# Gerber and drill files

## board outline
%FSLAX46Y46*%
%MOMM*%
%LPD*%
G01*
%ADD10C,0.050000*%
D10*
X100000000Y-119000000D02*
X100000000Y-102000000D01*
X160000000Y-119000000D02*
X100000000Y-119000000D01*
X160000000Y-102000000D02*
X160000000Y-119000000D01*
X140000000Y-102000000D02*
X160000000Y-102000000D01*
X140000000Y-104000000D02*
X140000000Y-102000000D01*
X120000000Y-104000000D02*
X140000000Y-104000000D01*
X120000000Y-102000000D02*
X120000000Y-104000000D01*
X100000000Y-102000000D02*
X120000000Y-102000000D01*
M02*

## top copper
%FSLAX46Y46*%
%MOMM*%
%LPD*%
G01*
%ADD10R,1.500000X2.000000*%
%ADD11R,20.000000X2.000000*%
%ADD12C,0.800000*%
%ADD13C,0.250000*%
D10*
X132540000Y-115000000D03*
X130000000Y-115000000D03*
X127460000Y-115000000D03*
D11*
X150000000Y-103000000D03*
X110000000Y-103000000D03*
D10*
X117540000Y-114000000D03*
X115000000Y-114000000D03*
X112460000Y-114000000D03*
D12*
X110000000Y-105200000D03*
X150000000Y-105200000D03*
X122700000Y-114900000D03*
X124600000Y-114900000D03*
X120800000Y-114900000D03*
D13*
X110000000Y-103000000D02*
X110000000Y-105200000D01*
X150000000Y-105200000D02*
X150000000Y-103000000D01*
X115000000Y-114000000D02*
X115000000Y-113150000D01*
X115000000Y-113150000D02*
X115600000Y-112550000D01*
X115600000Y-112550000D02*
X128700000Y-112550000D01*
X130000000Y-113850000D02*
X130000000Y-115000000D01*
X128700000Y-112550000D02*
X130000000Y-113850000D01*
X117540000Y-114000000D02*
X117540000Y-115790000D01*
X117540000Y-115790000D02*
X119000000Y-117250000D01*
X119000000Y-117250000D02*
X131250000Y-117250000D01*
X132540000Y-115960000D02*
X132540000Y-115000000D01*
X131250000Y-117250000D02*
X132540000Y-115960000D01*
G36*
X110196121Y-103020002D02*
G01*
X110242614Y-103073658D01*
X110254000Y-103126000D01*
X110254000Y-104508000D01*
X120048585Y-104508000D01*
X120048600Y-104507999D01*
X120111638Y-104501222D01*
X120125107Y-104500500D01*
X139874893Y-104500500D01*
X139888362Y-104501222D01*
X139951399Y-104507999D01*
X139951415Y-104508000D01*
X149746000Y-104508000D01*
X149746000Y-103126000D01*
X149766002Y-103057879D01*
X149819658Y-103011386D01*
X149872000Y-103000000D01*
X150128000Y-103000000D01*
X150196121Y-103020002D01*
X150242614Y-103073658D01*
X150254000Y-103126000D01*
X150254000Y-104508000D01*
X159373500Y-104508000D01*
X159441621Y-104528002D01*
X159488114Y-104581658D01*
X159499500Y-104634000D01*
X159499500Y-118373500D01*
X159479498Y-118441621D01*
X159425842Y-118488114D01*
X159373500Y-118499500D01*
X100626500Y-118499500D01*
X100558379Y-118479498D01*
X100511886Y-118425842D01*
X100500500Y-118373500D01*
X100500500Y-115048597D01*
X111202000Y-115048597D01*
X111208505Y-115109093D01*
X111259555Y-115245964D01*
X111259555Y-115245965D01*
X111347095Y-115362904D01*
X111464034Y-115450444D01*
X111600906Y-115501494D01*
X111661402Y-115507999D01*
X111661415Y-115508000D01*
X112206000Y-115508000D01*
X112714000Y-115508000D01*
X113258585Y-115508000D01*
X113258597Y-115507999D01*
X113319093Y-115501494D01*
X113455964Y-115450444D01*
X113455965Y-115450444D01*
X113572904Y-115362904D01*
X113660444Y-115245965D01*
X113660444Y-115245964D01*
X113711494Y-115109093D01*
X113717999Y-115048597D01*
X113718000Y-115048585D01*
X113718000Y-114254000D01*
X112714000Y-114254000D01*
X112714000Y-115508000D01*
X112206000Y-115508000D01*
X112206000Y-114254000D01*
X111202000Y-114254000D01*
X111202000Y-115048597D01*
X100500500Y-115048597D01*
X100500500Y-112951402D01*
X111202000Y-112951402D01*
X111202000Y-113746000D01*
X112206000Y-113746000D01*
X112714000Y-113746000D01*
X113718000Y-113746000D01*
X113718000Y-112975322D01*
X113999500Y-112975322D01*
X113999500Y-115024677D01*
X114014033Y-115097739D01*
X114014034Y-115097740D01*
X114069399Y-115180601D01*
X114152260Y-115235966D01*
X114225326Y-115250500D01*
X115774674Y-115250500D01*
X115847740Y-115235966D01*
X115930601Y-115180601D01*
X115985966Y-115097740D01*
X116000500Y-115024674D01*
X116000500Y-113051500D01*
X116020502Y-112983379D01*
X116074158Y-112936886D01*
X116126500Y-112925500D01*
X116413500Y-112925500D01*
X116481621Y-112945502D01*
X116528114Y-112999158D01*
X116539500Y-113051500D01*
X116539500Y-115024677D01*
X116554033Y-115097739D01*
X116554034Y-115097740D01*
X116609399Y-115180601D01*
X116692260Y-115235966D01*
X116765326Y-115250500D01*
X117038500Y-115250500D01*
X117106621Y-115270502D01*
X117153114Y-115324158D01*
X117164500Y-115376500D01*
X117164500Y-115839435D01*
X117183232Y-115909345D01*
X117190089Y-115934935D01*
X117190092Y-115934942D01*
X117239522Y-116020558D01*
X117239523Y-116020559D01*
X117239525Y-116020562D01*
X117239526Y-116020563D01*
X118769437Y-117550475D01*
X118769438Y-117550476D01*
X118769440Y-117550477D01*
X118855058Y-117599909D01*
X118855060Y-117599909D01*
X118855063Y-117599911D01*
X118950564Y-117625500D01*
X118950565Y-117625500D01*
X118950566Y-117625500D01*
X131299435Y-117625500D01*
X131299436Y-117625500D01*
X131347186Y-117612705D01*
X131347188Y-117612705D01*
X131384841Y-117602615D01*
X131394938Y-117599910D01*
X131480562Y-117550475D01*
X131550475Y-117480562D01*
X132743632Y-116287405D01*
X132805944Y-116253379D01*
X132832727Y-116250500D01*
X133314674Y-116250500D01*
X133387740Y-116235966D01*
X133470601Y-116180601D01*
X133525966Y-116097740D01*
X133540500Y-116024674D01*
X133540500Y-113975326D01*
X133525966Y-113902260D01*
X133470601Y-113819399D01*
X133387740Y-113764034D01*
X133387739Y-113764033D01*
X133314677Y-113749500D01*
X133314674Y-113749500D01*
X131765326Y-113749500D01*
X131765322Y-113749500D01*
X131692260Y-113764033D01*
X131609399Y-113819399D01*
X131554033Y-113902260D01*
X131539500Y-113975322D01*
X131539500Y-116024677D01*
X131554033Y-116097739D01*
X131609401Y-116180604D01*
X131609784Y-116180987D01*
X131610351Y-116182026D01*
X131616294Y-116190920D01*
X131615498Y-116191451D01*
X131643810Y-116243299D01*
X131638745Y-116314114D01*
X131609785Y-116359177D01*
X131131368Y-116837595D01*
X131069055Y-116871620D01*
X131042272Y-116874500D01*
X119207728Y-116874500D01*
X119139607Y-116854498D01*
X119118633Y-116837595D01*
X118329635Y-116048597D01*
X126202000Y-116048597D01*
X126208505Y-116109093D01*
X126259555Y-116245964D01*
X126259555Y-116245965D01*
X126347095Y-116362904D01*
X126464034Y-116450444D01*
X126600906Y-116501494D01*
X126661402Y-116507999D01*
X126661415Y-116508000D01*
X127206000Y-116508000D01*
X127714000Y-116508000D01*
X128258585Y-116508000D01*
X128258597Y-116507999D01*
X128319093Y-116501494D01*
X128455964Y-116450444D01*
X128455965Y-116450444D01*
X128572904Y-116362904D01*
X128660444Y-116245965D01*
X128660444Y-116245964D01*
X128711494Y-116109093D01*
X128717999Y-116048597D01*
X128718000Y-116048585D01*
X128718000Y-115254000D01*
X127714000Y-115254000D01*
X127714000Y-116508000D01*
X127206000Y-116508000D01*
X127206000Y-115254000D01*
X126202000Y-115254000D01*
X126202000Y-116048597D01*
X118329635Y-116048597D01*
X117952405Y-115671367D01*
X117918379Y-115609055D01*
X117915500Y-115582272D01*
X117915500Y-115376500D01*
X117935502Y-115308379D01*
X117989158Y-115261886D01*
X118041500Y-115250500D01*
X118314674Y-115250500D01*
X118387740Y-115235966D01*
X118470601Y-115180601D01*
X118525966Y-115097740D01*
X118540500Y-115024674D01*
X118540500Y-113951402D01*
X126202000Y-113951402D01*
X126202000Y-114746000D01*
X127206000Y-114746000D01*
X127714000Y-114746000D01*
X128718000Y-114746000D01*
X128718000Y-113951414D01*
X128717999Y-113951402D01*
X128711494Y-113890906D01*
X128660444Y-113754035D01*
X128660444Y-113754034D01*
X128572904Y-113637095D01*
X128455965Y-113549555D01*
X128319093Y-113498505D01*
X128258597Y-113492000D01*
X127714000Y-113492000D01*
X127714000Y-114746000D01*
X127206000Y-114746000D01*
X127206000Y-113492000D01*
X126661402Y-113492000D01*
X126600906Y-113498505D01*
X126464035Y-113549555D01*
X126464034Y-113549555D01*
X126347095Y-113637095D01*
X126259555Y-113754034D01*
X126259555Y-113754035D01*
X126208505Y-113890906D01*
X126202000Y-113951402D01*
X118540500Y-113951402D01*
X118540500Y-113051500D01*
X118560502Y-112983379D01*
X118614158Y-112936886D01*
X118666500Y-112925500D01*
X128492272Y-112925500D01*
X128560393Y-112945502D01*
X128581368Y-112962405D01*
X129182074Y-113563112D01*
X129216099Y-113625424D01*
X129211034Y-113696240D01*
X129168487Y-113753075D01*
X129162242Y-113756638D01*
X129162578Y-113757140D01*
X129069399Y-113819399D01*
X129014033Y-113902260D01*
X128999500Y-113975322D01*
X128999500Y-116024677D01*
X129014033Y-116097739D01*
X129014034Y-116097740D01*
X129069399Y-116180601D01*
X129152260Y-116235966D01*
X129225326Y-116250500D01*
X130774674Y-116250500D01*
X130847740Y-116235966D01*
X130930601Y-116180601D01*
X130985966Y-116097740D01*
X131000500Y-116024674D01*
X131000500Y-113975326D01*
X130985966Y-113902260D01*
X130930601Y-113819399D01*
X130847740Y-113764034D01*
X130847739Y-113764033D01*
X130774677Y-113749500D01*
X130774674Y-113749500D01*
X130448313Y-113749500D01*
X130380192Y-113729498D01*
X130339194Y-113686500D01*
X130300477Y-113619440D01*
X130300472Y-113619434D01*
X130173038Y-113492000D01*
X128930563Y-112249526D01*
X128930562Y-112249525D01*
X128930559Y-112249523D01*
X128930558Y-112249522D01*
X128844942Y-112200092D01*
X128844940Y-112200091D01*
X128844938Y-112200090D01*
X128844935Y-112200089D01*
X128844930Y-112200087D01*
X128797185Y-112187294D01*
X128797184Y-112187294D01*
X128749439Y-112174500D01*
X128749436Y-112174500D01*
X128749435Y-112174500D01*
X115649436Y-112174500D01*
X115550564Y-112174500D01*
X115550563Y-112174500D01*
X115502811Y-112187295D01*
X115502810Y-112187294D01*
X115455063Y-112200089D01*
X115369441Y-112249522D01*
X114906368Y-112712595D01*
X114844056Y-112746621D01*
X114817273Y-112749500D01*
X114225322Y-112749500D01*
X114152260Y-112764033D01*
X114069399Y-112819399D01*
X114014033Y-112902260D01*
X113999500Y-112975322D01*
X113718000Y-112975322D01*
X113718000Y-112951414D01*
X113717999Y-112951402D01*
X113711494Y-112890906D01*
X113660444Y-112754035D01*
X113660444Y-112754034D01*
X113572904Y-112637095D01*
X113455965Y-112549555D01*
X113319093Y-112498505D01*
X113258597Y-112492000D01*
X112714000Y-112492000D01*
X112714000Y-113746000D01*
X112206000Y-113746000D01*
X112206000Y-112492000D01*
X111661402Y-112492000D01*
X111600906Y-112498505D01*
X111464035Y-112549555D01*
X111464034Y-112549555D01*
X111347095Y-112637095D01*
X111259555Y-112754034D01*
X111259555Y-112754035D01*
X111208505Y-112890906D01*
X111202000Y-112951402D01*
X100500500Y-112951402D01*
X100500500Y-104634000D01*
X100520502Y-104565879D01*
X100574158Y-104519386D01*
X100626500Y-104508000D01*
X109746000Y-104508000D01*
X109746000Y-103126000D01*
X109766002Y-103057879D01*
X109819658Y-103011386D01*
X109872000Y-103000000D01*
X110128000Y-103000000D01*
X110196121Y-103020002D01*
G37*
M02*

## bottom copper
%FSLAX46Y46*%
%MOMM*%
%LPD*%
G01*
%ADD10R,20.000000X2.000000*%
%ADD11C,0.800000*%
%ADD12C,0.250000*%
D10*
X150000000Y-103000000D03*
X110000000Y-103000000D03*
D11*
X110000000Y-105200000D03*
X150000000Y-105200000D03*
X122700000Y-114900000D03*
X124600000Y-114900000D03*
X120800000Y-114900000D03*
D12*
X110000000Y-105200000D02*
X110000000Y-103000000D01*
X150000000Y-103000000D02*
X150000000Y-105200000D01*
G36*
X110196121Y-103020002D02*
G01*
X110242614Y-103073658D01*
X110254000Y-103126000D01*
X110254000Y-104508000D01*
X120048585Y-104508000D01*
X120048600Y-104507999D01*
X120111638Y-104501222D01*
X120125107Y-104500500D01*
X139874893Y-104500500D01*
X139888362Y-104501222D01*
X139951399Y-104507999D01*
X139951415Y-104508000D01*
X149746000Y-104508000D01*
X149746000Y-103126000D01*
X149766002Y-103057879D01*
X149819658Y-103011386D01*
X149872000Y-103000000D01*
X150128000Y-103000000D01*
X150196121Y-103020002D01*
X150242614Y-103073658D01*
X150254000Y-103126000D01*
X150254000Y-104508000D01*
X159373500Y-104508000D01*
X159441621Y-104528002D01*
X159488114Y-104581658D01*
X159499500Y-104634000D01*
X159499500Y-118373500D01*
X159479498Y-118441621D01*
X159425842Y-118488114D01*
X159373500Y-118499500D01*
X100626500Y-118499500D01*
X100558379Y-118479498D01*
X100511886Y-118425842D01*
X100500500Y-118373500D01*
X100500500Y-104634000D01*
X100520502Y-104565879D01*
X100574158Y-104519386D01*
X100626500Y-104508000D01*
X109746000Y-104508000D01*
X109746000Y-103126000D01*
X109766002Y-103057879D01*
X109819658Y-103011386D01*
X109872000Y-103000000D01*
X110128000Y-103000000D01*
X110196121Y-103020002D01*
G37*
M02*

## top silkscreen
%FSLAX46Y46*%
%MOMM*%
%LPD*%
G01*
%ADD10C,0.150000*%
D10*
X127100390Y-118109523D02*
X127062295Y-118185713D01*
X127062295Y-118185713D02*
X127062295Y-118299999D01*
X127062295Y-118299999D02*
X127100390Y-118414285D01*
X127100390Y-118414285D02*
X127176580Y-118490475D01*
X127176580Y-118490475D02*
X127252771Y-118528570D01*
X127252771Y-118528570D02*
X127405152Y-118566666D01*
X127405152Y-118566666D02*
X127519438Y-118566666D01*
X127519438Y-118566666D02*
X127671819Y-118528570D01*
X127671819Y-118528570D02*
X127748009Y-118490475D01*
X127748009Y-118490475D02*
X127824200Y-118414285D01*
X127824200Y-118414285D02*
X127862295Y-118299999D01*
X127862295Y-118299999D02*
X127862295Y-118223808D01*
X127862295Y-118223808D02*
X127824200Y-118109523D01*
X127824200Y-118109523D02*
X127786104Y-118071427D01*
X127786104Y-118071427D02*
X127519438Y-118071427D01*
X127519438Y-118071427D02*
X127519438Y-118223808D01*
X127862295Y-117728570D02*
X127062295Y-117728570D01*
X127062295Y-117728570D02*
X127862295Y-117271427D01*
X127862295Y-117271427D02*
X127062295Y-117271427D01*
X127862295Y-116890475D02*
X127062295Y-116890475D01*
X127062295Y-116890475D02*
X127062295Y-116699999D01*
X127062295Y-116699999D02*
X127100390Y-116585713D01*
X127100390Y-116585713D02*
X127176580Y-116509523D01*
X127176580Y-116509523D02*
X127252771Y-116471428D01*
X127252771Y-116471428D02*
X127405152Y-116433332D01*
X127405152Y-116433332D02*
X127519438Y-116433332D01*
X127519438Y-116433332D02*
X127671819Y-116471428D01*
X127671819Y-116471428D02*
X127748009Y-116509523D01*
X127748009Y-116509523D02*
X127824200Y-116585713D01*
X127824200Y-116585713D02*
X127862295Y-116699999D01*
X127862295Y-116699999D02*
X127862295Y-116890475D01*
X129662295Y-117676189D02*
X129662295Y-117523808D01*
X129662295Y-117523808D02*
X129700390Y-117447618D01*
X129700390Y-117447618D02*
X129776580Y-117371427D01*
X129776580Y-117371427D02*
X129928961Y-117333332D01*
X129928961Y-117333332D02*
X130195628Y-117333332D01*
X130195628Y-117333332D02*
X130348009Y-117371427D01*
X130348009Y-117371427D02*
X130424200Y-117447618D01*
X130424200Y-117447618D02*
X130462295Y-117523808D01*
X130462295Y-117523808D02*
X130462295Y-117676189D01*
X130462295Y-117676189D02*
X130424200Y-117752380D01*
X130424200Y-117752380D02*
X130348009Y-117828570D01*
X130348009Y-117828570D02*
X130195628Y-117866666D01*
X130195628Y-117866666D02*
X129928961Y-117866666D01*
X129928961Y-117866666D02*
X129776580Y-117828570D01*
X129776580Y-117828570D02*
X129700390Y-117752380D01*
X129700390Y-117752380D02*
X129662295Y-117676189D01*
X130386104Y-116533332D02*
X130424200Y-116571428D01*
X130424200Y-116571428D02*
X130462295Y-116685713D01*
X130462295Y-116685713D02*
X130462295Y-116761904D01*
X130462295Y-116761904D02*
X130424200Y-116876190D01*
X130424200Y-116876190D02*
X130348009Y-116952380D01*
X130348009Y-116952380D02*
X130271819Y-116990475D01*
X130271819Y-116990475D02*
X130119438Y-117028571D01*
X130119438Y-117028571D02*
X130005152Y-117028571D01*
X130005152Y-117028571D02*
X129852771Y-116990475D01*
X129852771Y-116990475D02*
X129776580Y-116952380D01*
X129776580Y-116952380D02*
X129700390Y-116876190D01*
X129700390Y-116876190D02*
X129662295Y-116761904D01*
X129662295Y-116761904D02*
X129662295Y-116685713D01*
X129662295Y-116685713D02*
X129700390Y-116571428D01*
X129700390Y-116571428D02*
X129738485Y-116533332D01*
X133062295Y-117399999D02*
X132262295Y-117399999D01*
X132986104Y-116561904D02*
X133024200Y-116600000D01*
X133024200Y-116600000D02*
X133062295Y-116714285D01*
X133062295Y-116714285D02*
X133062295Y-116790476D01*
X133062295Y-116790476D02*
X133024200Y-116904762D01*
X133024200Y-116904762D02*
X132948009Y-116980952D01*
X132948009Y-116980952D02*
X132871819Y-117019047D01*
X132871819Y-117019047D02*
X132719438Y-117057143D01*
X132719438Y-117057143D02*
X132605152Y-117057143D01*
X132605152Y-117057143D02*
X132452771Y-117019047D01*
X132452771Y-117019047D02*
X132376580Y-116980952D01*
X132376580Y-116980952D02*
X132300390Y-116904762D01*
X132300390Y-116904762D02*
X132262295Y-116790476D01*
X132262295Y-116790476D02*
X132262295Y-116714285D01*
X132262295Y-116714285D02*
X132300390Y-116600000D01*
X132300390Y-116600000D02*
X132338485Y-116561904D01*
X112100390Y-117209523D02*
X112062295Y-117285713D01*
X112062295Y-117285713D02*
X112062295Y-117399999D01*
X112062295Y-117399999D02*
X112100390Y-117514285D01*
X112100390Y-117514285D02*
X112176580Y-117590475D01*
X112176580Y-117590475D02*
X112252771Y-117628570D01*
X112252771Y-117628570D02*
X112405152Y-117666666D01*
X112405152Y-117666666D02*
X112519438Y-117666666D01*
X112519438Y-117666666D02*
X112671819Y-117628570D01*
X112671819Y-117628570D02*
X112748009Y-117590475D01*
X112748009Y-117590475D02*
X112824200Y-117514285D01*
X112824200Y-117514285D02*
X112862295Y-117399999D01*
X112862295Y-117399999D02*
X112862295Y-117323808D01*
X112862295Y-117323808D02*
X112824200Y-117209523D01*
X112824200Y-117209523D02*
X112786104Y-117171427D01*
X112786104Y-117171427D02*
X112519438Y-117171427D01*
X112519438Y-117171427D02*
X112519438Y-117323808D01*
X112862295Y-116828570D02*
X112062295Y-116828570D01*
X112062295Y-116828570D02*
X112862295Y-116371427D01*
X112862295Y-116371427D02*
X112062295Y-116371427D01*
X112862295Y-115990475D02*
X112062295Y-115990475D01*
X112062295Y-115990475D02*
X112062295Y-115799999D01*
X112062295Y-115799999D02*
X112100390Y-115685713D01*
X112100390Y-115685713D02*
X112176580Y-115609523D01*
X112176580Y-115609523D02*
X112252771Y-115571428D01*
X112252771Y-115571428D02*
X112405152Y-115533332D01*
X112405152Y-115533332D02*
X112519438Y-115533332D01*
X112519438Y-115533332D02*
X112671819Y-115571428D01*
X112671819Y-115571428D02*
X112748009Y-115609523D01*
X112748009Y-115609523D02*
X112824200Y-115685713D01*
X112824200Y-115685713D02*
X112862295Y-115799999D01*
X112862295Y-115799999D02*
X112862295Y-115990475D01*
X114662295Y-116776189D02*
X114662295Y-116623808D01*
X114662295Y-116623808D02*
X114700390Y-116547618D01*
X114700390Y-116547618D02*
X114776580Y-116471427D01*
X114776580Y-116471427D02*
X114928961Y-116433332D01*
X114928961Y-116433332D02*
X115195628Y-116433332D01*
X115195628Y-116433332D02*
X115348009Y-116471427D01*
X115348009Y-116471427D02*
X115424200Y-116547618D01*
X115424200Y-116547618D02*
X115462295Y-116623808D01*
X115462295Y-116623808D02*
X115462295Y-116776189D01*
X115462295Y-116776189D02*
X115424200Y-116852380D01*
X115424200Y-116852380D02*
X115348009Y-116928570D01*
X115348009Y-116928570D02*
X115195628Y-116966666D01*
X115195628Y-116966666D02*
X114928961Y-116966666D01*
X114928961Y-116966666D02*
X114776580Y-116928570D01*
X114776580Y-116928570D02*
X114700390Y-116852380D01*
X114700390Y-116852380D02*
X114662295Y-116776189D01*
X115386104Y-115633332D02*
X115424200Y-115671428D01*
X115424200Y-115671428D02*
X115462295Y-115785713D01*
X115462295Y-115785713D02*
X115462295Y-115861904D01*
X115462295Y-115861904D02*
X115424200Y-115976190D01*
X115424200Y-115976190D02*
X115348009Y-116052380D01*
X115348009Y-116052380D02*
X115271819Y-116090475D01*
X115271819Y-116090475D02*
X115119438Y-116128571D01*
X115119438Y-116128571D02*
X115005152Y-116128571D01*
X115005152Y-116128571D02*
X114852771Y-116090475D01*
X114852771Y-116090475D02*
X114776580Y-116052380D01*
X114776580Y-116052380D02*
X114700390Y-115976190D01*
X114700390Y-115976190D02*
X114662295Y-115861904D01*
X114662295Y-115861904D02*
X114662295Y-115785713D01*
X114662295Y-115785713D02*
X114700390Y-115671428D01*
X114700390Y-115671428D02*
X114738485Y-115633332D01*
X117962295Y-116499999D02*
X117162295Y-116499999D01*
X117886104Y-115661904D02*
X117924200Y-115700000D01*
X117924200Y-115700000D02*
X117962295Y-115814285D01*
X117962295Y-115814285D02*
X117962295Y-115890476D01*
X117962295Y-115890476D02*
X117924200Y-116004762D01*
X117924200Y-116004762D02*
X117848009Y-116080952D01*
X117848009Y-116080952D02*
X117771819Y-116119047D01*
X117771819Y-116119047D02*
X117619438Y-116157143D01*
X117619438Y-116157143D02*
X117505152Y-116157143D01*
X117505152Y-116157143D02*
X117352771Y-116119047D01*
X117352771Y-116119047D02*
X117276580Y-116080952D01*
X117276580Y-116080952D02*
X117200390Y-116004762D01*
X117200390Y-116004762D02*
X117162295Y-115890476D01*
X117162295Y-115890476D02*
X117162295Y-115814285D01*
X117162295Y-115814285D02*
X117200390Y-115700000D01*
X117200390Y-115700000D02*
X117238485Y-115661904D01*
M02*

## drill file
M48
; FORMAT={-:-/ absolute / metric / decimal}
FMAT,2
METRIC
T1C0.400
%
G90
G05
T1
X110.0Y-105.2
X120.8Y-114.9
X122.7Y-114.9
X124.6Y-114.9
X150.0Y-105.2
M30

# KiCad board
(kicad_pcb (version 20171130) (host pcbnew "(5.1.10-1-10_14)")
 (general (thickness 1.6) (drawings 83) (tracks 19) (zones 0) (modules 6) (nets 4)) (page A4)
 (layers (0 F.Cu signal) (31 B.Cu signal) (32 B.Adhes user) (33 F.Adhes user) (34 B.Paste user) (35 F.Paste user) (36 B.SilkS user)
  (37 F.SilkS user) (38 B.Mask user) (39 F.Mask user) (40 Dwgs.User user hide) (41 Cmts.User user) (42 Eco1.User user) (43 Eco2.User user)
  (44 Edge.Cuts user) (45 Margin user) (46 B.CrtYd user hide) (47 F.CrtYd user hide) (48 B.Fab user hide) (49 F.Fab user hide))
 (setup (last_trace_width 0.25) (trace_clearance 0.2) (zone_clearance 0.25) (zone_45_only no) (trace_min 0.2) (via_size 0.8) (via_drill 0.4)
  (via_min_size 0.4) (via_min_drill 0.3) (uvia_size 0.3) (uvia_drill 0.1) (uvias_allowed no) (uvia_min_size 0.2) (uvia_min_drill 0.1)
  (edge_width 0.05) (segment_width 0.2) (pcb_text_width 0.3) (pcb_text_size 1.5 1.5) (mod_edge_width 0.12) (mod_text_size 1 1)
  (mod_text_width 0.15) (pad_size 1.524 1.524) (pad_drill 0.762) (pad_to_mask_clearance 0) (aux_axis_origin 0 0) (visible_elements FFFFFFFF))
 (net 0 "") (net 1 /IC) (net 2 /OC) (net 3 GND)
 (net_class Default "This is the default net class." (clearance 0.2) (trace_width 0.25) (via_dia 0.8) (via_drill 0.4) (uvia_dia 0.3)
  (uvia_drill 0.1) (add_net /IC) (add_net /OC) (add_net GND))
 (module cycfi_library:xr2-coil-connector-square (layer F.Cu) (at 130 115)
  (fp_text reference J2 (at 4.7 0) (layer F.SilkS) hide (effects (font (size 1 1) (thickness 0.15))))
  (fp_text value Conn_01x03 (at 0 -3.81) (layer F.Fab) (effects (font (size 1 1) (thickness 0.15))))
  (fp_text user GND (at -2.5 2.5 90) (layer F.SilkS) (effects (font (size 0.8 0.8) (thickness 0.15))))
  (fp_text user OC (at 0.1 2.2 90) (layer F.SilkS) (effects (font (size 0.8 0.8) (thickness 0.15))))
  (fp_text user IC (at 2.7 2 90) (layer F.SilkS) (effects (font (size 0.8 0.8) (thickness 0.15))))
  (pad 3 smd rect (at 2.54 0) (size 1.5 2) (layers F.Cu F.Paste F.Mask) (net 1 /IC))
  (pad 2 smd rect (at 0 0) (size 1.5 2) (layers F.Cu F.Paste F.Mask) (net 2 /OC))
  (pad 1 smd rect (at -2.54 0) (size 1.5 2) (layers F.Cu F.Paste F.Mask) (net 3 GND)))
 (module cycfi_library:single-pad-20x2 (layer B.Cu) (at 150 103)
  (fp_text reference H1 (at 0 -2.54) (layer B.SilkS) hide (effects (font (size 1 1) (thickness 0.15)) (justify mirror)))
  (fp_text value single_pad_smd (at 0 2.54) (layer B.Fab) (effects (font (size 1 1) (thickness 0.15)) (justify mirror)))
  (pad 1 smd rect (at 0 0) (size 20 2) (layers B.Cu B.Paste B.Mask) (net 3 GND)))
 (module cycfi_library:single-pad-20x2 (layer F.Cu) (at 150 103)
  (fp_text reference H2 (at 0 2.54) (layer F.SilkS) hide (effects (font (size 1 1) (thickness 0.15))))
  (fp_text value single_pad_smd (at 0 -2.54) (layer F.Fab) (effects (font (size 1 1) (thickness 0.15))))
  (pad 1 smd rect (at 0 0) (size 20 2) (layers F.Cu F.Paste F.Mask) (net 3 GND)))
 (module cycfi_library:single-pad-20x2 (layer B.Cu) (at 110 103)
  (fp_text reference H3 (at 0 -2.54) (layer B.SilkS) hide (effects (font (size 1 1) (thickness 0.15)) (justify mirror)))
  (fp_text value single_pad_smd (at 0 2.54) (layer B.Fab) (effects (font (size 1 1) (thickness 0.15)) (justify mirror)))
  (pad 1 smd rect (at 0 0) (size 20 2) (layers B.Cu B.Paste B.Mask) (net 3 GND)))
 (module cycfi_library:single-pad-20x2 (layer F.Cu) (at 110 103)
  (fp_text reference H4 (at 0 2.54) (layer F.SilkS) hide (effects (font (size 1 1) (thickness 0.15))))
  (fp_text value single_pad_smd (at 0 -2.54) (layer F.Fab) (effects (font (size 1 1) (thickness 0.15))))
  (pad 1 smd rect (at 0 0) (size 20 2) (layers F.Cu F.Paste F.Mask) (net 3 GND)))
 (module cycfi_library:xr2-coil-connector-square (layer F.Cu) (at 115 114)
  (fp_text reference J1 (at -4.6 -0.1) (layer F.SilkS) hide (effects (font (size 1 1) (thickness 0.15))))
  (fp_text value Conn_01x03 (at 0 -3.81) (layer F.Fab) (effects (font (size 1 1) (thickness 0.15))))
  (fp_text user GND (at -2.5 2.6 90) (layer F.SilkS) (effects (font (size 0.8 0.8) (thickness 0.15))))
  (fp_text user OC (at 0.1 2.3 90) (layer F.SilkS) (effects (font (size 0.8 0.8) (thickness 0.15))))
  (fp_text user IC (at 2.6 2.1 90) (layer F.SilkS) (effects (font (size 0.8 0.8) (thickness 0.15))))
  (pad 3 smd rect (at 2.54 0) (size 1.5 2) (layers F.Cu F.Paste F.Mask) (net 1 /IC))
  (pad 2 smd rect (at 0 0) (size 1.5 2) (layers F.Cu F.Paste F.Mask) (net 2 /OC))
  (pad 1 smd rect (at -2.54 0) (size 1.5 2) (layers F.Cu F.Paste F.Mask) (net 3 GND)))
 (gr_line (start 100 119) (end 100 102) (layer Edge.Cuts) (width 0.05))
 (gr_line (start 160 119) (end 100 119) (layer Edge.Cuts) (width 0.05))
 (gr_line (start 160 102) (end 160 119) (layer Edge.Cuts) (width 0.05))
 (gr_line (start 140 102) (end 160 102) (layer Edge.Cuts) (width 0.05))
 (gr_line (start 140 104) (end 140 102) (layer Edge.Cuts) (width 0.05))
 (gr_line (start 120 104) (end 140 104) (layer Edge.Cuts) (width 0.05))
 (gr_line (start 120 102) (end 120 104) (layer Edge.Cuts) (width 0.05))
 (gr_line (start 100 102) (end 120 102) (layer Edge.Cuts) (width 0.05))
 (via (at 110 105.2) (size 0.8) (drill 0.4) (layers F.Cu B.Cu) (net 3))
 (segment (start 110 103) (end 110 105.2) (width 0.25) (layer F.Cu) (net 3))
 (segment (start 110 105.2) (end 110 103) (width 0.25) (layer B.Cu) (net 3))
 (via (at 150 105.2) (size 0.8) (drill 0.4) (layers F.Cu B.Cu) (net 3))
 (segment (start 150 103) (end 150 105.2) (width 0.25) (layer B.Cu) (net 3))
 (segment (start 150 105.2) (end 150 103) (width 0.25) (layer F.Cu) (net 3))
 (via (at 122.7 114.9) (size 0.8) (drill 0.4) (layers F.Cu B.Cu) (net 3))
 (via (at 124.6 114.9) (size 0.8) (drill 0.4) (layers F.Cu B.Cu) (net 3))
 (via (at 120.8 114.9) (size 0.8) (drill 0.4) (layers F.Cu B.Cu) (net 3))
 (segment (start 115 114) (end 115 113.15) (width 0.25) (layer F.Cu) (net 2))
 (segment (start 115 113.15) (end 115.6 112.55) (width 0.25) (layer F.Cu) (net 2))
 (segment (start 115.6 112.55) (end 128.7 112.55) (width 0.25) (layer F.Cu) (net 2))
 (segment (start 130 113.85) (end 130 115) (width 0.25) (layer F.Cu) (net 2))
 (segment (start 128.7 112.55) (end 130 113.85) (width 0.25) (layer F.Cu) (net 2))
 (segment (start 117.54 114) (end 117.54 115.79) (width 0.25) (layer F.Cu) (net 1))
 (segment (start 117.54 115.79) (end 119 117.25) (width 0.25) (layer F.Cu) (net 1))
 (segment (start 119 117.25) (end 131.25 117.25) (width 0.25) (layer F.Cu) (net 1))
 (segment (start 132.54 115.96) (end 132.54 115) (width 0.25) (layer F.Cu) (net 1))
 (segment (start 131.25 117.25) (end 132.54 115.96) (width 0.25) (layer F.Cu) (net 1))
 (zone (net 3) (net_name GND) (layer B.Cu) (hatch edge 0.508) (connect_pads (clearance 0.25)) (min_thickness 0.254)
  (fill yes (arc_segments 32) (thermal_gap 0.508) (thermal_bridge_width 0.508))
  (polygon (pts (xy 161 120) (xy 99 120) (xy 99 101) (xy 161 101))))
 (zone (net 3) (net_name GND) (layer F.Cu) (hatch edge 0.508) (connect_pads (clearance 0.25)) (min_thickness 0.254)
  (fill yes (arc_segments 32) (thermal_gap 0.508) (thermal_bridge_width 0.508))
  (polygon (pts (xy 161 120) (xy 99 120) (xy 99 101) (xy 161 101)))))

